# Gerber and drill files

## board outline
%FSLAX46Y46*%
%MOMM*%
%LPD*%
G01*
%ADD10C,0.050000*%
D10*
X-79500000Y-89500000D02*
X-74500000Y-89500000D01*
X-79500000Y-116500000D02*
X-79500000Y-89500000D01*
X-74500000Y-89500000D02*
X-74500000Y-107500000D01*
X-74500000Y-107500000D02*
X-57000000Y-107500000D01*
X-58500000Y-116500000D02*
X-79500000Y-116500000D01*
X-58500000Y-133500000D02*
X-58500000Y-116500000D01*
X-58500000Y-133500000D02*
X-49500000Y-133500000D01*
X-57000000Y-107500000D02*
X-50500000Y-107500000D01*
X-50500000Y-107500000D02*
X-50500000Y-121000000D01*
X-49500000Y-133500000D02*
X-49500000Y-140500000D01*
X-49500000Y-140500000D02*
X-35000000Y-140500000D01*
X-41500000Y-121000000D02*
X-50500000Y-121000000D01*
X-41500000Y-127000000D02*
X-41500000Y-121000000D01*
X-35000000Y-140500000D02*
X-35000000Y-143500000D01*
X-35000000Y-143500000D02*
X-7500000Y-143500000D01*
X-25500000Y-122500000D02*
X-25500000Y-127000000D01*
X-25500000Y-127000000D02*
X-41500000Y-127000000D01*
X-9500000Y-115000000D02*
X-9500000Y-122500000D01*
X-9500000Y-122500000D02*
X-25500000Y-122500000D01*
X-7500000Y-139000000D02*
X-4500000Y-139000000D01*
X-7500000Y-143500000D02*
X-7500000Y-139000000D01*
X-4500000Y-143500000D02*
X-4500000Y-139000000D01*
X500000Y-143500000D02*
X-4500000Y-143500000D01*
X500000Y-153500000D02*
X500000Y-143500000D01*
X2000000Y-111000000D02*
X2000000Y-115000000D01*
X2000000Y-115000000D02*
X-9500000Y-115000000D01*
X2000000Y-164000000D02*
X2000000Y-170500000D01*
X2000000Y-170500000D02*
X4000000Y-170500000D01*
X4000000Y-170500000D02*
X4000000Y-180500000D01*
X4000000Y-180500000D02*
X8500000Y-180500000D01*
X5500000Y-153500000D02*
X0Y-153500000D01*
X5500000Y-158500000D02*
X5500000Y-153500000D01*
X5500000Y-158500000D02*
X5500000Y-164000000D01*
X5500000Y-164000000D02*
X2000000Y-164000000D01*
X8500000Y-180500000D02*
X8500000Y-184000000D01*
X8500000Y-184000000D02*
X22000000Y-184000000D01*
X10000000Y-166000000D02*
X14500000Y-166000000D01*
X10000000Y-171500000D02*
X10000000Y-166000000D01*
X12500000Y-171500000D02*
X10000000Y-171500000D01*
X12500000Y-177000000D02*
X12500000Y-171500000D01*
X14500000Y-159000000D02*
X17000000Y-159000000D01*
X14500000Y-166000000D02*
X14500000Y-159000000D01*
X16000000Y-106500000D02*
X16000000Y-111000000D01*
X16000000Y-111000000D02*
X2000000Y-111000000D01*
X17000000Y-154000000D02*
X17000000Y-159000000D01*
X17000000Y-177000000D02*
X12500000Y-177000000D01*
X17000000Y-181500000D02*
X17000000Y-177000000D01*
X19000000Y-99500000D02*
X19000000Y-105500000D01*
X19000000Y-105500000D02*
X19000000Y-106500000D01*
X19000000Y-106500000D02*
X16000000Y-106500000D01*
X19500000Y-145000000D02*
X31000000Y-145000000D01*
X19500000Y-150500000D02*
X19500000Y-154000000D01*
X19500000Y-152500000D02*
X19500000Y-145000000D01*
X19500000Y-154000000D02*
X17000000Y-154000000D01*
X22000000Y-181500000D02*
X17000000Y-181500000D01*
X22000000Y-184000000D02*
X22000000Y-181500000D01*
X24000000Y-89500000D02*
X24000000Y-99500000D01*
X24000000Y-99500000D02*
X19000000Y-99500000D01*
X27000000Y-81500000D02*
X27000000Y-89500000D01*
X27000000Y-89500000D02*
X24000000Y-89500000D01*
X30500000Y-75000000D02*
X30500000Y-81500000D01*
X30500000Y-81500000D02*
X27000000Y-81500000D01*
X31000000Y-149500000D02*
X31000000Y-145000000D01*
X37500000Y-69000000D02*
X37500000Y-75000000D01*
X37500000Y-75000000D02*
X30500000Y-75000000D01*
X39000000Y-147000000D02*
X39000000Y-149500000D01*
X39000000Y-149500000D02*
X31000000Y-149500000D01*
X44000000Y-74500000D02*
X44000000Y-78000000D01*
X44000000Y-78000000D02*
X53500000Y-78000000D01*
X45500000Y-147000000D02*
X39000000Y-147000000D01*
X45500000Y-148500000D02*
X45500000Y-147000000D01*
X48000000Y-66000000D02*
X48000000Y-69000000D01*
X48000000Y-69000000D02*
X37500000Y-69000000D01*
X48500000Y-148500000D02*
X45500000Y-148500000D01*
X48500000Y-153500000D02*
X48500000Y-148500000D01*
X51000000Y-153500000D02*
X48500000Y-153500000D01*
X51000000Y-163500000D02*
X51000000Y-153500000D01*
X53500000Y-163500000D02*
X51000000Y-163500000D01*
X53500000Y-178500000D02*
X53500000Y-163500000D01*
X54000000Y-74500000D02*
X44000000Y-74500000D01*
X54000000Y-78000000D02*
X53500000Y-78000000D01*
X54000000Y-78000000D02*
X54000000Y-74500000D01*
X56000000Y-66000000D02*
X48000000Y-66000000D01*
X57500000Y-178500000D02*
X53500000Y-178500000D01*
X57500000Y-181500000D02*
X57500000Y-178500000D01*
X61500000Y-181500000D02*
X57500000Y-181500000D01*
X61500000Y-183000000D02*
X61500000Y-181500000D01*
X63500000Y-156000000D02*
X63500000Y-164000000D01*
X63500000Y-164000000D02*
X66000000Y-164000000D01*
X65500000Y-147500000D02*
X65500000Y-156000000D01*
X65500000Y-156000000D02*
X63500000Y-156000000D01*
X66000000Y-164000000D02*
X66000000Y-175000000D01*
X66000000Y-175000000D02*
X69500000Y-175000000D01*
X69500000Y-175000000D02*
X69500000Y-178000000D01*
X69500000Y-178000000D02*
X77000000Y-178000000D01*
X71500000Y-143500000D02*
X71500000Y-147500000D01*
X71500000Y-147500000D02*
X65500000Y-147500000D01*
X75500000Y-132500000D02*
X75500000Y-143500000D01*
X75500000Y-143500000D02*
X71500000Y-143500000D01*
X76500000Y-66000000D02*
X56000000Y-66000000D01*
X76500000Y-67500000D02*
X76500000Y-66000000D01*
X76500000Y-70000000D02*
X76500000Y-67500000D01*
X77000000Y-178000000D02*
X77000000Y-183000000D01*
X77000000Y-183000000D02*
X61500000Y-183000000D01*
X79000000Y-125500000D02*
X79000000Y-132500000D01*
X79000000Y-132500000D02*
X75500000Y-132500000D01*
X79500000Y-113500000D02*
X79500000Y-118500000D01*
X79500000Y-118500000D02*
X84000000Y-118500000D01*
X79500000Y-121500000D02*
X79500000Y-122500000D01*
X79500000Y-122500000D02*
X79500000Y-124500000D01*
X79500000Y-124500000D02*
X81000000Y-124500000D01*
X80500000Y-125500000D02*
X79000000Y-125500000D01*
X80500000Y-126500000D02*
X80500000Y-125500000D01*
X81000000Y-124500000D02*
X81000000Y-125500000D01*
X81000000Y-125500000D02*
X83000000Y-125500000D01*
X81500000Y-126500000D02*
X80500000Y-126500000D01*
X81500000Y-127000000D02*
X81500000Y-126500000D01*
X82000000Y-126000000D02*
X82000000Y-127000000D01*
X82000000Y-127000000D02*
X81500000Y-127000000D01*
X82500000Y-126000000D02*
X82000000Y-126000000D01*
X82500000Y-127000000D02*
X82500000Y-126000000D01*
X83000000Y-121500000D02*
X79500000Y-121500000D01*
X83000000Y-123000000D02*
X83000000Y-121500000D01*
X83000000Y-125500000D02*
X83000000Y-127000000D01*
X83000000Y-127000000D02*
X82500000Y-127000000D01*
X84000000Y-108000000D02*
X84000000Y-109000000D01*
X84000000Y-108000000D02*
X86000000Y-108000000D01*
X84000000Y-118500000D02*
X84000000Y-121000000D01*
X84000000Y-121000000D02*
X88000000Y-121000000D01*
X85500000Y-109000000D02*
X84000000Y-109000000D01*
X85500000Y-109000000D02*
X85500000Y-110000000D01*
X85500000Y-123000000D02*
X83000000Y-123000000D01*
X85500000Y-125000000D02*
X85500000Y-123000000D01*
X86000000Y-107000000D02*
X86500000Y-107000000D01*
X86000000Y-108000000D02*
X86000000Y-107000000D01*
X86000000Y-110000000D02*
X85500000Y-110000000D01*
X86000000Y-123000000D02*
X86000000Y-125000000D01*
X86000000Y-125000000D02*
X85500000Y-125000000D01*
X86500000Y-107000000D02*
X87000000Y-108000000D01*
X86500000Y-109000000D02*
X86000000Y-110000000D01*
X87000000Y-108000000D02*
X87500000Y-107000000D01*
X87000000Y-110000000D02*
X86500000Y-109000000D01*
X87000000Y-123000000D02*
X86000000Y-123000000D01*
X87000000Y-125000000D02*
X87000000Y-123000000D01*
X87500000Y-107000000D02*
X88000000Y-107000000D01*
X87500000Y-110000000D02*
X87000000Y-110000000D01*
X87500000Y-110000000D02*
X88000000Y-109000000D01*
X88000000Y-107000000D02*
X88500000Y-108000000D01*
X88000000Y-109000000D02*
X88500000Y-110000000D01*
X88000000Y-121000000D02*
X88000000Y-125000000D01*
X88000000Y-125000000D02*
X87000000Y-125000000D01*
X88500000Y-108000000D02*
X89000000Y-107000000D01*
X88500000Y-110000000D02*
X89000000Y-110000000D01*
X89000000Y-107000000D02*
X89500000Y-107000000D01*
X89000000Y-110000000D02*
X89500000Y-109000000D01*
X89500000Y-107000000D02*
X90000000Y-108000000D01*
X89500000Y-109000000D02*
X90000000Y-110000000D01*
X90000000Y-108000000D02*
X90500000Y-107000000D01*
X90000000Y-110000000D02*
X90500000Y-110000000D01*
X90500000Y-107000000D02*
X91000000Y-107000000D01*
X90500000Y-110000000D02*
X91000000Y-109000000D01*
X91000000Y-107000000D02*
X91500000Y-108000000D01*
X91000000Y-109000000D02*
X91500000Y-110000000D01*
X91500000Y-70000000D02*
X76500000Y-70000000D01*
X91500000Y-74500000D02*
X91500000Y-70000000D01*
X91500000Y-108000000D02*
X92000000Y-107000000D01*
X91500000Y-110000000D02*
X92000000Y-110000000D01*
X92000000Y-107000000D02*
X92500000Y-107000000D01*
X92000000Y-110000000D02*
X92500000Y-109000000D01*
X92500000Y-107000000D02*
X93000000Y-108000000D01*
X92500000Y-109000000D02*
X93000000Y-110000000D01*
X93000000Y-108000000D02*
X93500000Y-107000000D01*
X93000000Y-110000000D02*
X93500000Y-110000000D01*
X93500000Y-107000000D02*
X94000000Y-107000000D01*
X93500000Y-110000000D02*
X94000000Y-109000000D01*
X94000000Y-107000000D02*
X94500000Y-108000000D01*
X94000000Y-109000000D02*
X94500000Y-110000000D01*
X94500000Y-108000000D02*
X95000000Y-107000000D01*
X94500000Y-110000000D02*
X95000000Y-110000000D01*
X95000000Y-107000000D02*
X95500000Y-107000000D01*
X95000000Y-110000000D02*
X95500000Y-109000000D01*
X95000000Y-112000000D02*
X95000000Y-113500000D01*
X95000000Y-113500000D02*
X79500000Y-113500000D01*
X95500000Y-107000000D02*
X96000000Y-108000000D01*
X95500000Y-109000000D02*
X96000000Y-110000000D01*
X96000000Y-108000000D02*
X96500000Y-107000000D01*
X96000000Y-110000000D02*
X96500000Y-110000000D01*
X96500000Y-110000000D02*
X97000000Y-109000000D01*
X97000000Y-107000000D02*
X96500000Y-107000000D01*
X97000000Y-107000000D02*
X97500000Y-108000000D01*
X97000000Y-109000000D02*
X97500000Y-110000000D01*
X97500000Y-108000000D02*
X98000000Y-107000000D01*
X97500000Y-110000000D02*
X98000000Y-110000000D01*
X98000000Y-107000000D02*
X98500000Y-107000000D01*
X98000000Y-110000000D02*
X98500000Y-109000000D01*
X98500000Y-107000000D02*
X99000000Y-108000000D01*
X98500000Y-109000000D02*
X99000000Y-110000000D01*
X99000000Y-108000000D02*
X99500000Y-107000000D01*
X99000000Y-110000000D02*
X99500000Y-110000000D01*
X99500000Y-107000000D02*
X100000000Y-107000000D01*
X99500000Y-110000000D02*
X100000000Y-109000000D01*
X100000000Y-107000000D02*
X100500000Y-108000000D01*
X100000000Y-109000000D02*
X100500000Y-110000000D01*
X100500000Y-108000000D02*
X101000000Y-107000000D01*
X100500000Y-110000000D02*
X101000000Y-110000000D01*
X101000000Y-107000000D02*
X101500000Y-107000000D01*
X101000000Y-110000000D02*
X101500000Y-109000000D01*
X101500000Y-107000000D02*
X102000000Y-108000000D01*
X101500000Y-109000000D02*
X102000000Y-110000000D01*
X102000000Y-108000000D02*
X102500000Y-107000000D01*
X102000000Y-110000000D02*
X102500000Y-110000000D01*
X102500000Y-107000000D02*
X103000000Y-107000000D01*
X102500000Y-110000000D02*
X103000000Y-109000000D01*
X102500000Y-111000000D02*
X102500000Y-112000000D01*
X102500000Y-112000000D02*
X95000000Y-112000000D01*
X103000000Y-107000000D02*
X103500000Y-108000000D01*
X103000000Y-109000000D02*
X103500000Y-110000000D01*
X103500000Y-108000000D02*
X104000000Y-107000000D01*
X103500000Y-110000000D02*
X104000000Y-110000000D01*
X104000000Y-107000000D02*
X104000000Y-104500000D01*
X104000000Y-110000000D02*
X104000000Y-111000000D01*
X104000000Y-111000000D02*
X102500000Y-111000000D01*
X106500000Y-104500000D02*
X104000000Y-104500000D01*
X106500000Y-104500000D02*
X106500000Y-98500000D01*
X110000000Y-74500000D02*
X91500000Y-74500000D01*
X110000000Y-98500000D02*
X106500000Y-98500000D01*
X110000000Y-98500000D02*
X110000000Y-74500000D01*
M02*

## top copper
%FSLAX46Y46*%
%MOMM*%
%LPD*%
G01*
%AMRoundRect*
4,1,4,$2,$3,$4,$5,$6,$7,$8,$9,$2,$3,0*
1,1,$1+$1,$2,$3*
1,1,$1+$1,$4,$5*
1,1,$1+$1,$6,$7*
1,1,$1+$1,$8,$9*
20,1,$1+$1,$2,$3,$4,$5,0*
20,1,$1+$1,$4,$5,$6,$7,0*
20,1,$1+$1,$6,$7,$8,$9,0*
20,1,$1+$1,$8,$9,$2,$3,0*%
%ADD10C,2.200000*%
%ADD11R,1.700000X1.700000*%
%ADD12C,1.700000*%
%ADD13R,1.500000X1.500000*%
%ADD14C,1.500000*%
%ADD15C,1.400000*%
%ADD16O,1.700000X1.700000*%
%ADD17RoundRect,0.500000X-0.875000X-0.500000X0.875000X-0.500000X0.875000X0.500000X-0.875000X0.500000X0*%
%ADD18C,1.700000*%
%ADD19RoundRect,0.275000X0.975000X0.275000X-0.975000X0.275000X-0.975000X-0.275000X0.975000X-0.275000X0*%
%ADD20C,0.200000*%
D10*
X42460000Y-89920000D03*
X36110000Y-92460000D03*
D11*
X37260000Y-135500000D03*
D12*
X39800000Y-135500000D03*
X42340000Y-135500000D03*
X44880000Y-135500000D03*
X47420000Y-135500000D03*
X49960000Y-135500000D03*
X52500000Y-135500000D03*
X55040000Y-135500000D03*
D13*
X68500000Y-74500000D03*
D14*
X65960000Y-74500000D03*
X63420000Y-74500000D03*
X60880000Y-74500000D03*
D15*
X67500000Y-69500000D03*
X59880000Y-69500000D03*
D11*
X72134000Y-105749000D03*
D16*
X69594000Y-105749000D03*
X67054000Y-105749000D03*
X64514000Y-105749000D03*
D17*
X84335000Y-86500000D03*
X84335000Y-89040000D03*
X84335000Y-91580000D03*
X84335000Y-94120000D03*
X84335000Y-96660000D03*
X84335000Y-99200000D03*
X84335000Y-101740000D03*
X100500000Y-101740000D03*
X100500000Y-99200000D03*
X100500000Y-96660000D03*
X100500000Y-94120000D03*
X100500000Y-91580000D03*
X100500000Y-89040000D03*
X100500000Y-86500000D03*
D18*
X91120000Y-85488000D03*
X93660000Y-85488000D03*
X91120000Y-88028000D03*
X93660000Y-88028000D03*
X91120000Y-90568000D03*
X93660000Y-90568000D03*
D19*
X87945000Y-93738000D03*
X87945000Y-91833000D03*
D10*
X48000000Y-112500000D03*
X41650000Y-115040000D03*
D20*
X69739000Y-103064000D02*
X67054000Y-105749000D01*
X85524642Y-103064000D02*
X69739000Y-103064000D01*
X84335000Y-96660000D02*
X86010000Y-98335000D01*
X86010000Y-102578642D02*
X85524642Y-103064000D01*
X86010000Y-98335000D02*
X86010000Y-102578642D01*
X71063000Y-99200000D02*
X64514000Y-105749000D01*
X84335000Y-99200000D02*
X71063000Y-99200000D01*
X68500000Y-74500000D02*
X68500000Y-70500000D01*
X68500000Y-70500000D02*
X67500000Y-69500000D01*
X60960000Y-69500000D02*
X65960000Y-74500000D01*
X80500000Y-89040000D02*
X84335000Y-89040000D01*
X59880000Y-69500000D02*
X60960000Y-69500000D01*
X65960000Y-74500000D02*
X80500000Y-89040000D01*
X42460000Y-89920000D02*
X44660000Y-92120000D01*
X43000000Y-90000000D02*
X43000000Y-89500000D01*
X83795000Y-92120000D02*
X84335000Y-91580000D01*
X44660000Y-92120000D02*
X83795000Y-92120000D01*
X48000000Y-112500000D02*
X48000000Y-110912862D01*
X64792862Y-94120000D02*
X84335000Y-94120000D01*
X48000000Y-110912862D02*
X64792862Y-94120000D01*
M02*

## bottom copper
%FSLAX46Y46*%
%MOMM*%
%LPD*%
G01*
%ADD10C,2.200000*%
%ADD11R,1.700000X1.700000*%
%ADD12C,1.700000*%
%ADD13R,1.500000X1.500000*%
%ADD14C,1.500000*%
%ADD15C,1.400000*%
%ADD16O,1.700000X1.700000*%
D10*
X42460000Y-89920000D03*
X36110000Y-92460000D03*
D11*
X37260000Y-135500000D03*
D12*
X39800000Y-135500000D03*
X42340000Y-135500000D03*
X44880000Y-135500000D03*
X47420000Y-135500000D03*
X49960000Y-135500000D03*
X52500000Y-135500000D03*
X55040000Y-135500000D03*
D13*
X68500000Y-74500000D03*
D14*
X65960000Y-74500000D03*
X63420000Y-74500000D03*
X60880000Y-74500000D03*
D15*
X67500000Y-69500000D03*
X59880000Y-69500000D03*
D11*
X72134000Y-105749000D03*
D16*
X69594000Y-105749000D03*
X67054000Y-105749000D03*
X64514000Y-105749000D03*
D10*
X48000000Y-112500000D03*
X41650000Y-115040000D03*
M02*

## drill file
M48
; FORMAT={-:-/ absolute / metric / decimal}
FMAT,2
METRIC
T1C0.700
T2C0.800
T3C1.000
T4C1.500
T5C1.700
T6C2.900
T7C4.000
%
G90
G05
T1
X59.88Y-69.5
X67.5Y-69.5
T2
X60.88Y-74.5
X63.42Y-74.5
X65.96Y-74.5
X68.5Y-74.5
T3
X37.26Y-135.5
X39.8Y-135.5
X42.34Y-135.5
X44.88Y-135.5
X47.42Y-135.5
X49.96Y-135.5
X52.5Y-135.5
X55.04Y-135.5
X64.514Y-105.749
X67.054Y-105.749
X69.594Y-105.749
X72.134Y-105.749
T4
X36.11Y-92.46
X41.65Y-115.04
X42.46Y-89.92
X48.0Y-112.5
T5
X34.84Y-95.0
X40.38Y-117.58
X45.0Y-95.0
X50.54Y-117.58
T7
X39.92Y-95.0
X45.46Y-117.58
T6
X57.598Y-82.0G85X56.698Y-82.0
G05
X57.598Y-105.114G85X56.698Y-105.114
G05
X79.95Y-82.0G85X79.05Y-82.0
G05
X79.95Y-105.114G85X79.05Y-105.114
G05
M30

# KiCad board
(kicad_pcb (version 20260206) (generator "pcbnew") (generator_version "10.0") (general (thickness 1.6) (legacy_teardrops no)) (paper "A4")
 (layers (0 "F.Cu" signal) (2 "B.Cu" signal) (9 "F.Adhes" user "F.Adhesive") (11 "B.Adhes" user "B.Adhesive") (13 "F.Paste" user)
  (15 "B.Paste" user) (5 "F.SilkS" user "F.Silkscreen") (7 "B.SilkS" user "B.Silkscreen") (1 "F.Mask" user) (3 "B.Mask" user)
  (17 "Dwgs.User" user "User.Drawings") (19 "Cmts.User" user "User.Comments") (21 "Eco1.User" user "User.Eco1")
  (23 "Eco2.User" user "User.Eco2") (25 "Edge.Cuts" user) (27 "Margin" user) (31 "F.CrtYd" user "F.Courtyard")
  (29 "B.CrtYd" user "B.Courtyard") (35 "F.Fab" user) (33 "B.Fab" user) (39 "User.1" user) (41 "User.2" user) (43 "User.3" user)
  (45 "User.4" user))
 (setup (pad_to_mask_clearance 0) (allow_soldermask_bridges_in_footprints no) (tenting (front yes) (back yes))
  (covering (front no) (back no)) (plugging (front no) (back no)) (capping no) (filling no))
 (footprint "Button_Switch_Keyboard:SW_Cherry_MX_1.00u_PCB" (layer "F.Cu") (at 42.46 89.92)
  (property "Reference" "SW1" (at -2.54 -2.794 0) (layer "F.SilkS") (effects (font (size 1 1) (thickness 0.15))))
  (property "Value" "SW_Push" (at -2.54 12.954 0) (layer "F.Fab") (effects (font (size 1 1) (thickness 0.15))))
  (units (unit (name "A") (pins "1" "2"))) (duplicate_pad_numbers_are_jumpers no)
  (pad "" np_thru_hole circle (at -7.62 5.08) (size 1.7 1.7) (drill 1.7) (layers "*.Cu" "*.Mask"))
  (pad "" np_thru_hole circle (at -2.54 5.08) (size 4 4) (drill 4) (layers "*.Cu" "*.Mask"))
  (pad "" np_thru_hole circle (at 2.54 5.08) (size 1.7 1.7) (drill 1.7) (layers "*.Cu" "*.Mask"))
  (pad "1" thru_hole circle (at 0 0) (size 2.2 2.2) (drill 1.5) (layers "*.Cu" "*.Mask") (remove_unused_layers no) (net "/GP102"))
  (pad "2" thru_hole circle (at -6.35 2.54) (size 2.2 2.2) (drill 1.5) (layers "*.Cu" "*.Mask") (remove_unused_layers no) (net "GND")))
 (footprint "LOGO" (layer "F.Cu") (at 22 131)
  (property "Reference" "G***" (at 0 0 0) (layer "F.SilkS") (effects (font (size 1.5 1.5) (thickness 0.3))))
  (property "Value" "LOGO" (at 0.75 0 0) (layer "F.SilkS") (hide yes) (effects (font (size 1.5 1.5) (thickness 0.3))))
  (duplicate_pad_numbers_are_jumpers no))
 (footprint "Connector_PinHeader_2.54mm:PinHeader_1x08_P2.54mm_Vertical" (layer "F.Cu") (at 37.26 135.5 90)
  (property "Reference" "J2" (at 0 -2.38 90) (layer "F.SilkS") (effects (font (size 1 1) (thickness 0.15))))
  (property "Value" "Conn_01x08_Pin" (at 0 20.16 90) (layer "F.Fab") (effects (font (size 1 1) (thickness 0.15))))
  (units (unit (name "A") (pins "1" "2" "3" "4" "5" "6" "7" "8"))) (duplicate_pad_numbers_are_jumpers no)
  (pad "1" thru_hole rect (at 0 0 90) (size 1.7 1.7) (drill 1) (layers "*.Cu" "*.Mask") (remove_unused_layers no) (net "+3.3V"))
  (pad "2" thru_hole circle (at 0 2.54 90) (size 1.7 1.7) (drill 1) (layers "*.Cu" "*.Mask") (remove_unused_layers no) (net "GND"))
  (pad "3" thru_hole circle (at 0 5.08 90) (size 1.7 1.7) (drill 1) (layers "*.Cu" "*.Mask") (remove_unused_layers no) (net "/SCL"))
  (pad "4" thru_hole circle (at 0 7.62 90) (size 1.7 1.7) (drill 1) (layers "*.Cu" "*.Mask") (remove_unused_layers no) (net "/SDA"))
  (pad "5" thru_hole circle (at 0 10.16 90) (size 1.7 1.7) (drill 1) (layers "*.Cu" "*.Mask") (remove_unused_layers no)
   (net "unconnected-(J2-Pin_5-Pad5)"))
  (pad "6" thru_hole circle (at 0 12.7 90) (size 1.7 1.7) (drill 1) (layers "*.Cu" "*.Mask") (remove_unused_layers no)
   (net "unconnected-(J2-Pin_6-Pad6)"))
  (pad "7" thru_hole circle (at 0 15.24 90) (size 1.7 1.7) (drill 1) (layers "*.Cu" "*.Mask") (remove_unused_layers no)
   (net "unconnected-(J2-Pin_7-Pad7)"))
  (pad "8" thru_hole circle (at 0 17.78 90) (size 1.7 1.7) (drill 1) (layers "*.Cu" "*.Mask") (remove_unused_layers no)
   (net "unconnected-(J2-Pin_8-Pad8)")))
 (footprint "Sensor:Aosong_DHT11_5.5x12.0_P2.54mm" (layer "F.Cu") (at 68.5 74.5 -90)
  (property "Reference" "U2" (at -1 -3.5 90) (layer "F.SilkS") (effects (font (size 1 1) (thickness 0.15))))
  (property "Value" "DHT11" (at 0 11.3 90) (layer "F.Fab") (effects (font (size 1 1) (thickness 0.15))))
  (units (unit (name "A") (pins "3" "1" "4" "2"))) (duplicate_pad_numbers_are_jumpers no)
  (pad "1" thru_hole rect (at 0 0 270) (size 1.5 1.5) (drill 0.8) (layers "*.Cu" "*.Mask") (remove_unused_layers no) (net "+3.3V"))
  (pad "2" thru_hole circle (at 0 2.54 270) (size 1.5 1.5) (drill 0.8) (layers "*.Cu" "*.Mask") (remove_unused_layers no)
   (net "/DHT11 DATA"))
  (pad "3" thru_hole circle (at 0 5.08 270) (size 1.5 1.5) (drill 0.8) (layers "*.Cu" "*.Mask") (remove_unused_layers no)
   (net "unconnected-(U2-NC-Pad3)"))
  (pad "4" thru_hole circle (at 0 7.62 270) (size 1.5 1.5) (drill 0.8) (layers "*.Cu" "*.Mask") (remove_unused_layers no) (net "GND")))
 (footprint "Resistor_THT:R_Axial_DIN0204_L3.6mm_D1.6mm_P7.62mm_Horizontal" (layer "F.Cu") (at 67.5 69.5 180)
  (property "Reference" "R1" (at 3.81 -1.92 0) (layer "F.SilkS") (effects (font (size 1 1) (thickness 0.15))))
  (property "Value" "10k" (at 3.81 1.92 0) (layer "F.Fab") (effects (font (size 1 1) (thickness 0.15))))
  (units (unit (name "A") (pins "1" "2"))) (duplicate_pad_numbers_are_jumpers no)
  (pad "1" thru_hole circle (at 0 0 180) (size 1.4 1.4) (drill 0.7) (layers "*.Cu" "*.Mask") (remove_unused_layers no) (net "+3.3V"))
  (pad "2" thru_hole circle (at 7.62 0 180) (size 1.4 1.4) (drill 0.7) (layers "*.Cu" "*.Mask") (remove_unused_layers no)
   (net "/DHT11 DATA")))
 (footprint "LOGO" (layer "F.Cu") (at 68.5 121.5)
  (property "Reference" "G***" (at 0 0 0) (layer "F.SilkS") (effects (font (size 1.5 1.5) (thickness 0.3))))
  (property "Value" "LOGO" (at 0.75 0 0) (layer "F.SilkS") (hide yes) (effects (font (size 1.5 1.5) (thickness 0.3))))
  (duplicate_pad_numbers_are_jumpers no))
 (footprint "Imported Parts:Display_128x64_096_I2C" (layer "F.Cu") (at 68.324 105.749 180)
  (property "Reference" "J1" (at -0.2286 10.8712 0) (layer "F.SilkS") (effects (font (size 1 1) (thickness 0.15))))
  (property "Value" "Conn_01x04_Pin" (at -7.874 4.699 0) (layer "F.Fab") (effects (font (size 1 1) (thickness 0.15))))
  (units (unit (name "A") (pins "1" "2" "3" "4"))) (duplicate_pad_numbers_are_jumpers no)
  (pad "" np_thru_hole oval (at -11.176 0.635 180) (size 3.8 2.9) (drill oval 3.8 2.9) (layers "*.Cu" "*.Mask"))
  (pad "" np_thru_hole oval (at -11.176 23.749 180) (size 3.8 2.9) (drill oval 3.8 2.9) (layers "*.Cu" "*.Mask"))
  (pad "" np_thru_hole oval (at 11.176 0.635 180) (size 3.8 2.9) (drill oval 3.8 2.9) (layers "*.Cu" "*.Mask"))
  (pad "" np_thru_hole oval (at 11.176 23.749 180) (size 3.8 2.9) (drill oval 3.8 2.9) (layers "*.Cu" "*.Mask"))
  (pad "1" thru_hole rect (at -3.81 0 270) (size 1.7 1.7) (drill 1) (layers "*.Cu" "*.Mask") (remove_unused_layers no) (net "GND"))
  (pad "2" thru_hole oval (at -1.27 0 270) (size 1.7 1.7) (drill 1) (layers "*.Cu" "*.Mask") (remove_unused_layers no) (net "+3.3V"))
  (pad "3" thru_hole oval (at 1.27 0 270) (size 1.7 1.7) (drill 1) (layers "*.Cu" "*.Mask") (remove_unused_layers no) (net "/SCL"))
  (pad "4" thru_hole oval (at 3.81 0 270) (size 1.7 1.7) (drill 1) (layers "*.Cu" "*.Mask") (remove_unused_layers no) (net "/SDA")))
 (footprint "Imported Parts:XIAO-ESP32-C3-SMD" (layer "F.Cu") (at 83.5 104.62)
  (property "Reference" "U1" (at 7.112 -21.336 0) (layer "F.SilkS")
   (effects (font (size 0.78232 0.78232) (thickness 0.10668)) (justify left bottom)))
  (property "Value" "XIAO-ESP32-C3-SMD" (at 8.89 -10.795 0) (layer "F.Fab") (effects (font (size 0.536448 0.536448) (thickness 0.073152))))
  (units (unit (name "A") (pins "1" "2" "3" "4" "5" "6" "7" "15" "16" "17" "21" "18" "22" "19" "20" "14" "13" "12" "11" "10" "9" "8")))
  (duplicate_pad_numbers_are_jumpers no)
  (pad "1" smd roundrect (at 0.835 -18.12) (size 2.75 2) (layers "F.Cu" "F.Mask" "F.Paste") (roundrect_rratio 0.25)
   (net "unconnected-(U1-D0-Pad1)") (solder_mask_margin 0.0508) (thermal_bridge_angle 45))
  (pad "2" smd roundrect (at 0.835 -15.58) (size 2.75 2) (layers "F.Cu" "F.Mask" "F.Paste") (roundrect_rratio 0.25) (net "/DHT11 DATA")
   (solder_mask_margin 0.0508) (thermal_bridge_angle 45))
  (pad "3" smd roundrect (at 0.835 -13.04) (size 2.75 2) (layers "F.Cu" "F.Mask" "F.Paste") (roundrect_rratio 0.25) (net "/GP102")
   (solder_mask_margin 0.0508) (thermal_bridge_angle 45))
  (pad "4" smd roundrect (at 0.835 -10.5) (size 2.75 2) (layers "F.Cu" "F.Mask" "F.Paste") (roundrect_rratio 0.25) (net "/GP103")
   (solder_mask_margin 0.0508) (thermal_bridge_angle 45))
  (pad "5" smd roundrect (at 0.835 -7.96) (size 2.75 2) (layers "F.Cu" "F.Mask" "F.Paste") (roundrect_rratio 0.25) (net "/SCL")
   (solder_mask_margin 0.0508) (thermal_bridge_angle 45))
  (pad "6" smd roundrect (at 0.835 -5.42) (size 2.75 2) (layers "F.Cu" "F.Mask" "F.Paste") (roundrect_rratio 0.25) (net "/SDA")
   (solder_mask_margin 0.0508) (thermal_bridge_angle 45))
  (pad "7" smd roundrect (at 0.835 -2.88) (size 2.75 2) (layers "F.Cu" "F.Mask" "F.Paste") (roundrect_rratio 0.25)
   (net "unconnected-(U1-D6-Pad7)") (solder_mask_margin 0.0508) (thermal_bridge_angle 45))
  (pad "8" smd roundrect (at 17 -2.88) (size 2.75 2) (layers "F.Cu" "F.Mask" "F.Paste") (roundrect_rratio 0.25)
   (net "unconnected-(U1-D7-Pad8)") (solder_mask_margin 0.0508) (thermal_bridge_angle 45))
  (pad "9" smd roundrect (at 17 -5.42) (size 2.75 2) (layers "F.Cu" "F.Mask" "F.Paste") (roundrect_rratio 0.25)
   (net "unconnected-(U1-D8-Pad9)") (solder_mask_margin 0.0508) (thermal_bridge_angle 45))
  (pad "10" smd roundrect (at 17 -7.96) (size 2.75 2) (layers "F.Cu" "F.Mask" "F.Paste") (roundrect_rratio 0.25)
   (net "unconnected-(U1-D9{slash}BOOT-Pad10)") (solder_mask_margin 0.0508) (thermal_bridge_angle 45))
  (pad "11" smd roundrect (at 17 -10.5) (size 2.75 2) (layers "F.Cu" "F.Mask" "F.Paste") (roundrect_rratio 0.25)
   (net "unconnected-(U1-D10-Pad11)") (solder_mask_margin 0.0508) (thermal_bridge_angle 45))
  (pad "12" smd roundrect (at 17 -13.04) (size 2.75 2) (layers "F.Cu" "F.Mask" "F.Paste") (roundrect_rratio 0.25) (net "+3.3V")
   (solder_mask_margin 0.0508) (thermal_bridge_angle 45))
  (pad "13" smd roundrect (at 17 -15.58) (size 2.75 2) (layers "F.Cu" "F.Mask" "F.Paste") (roundrect_rratio 0.25) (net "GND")
   (solder_mask_margin 0.0508) (thermal_bridge_angle 45))
  (pad "14" smd roundrect (at 17 -18.12) (size 2.75 2) (layers "F.Cu" "F.Mask" "F.Paste") (roundrect_rratio 0.25) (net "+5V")
   (solder_mask_margin 0.0508) (thermal_bridge_angle 45))
  (pad "15" smd circle (at 7.62 -19.132) (size 1.7 1.7) (layers "F.Cu" "F.Mask" "F.Paste") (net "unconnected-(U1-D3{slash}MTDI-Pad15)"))
  (pad "16" smd circle (at 10.16 -19.132) (size 1.7 1.7) (layers "F.Cu" "F.Mask" "F.Paste") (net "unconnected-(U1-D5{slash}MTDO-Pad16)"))
  (pad "17" smd circle (at 7.62 -16.592) (size 1.7 1.7) (layers "F.Cu" "F.Mask" "F.Paste") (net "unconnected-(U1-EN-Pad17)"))
  (pad "18" smd circle (at 10.16 -16.592) (size 1.7 1.7) (layers "F.Cu" "F.Mask" "F.Paste") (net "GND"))
  (pad "19" smd circle (at 7.62 -14.052) (size 1.7 1.7) (layers "F.Cu" "F.Mask" "F.Paste") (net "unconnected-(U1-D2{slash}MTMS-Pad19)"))
  (pad "20" smd circle (at 10.16 -14.052) (size 1.7 1.7) (layers "F.Cu" "F.Mask" "F.Paste") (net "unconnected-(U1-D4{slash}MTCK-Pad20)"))
  (pad "21" smd roundrect (at 4.445 -10.882 180) (size 2.5 1.1) (layers "F.Cu" "F.Mask" "F.Paste") (roundrect_rratio 0.25)
   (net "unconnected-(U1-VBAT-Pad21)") (thermal_bridge_angle 45))
  (pad "22" smd roundrect (at 4.445 -12.787 180) (size 2.5 1.1) (layers "F.Cu" "F.Mask" "F.Paste") (roundrect_rratio 0.25)
   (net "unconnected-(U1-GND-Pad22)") (thermal_bridge_angle 45)))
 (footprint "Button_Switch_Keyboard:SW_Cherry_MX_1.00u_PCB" (layer "F.Cu") (at 48 112.5)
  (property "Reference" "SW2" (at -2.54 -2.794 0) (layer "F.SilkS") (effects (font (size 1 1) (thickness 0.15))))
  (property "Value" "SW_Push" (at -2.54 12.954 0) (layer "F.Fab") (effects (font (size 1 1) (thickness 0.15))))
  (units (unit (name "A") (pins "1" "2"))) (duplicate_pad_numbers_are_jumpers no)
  (pad "" np_thru_hole circle (at -7.62 5.08) (size 1.7 1.7) (drill 1.7) (layers "*.Cu" "*.Mask"))
  (pad "" np_thru_hole circle (at -2.54 5.08) (size 4 4) (drill 4) (layers "*.Cu" "*.Mask"))
  (pad "" np_thru_hole circle (at 2.54 5.08) (size 1.7 1.7) (drill 1.7) (layers "*.Cu" "*.Mask"))
  (pad "1" thru_hole circle (at 0 0) (size 2.2 2.2) (drill 1.5) (layers "*.Cu" "*.Mask") (remove_unused_layers no) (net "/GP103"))
  (pad "2" thru_hole circle (at -6.35 2.54) (size 2.2 2.2) (drill 1.5) (layers "*.Cu" "*.Mask") (remove_unused_layers no) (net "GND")))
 (gr_line (start -79.5 89.5) (end -74.5 89.5) (stroke (width 0.05) (type default)) (layer "Edge.Cuts"))
 (gr_line (start -79.5 116.5) (end -79.5 89.5) (stroke (width 0.05) (type default)) (layer "Edge.Cuts"))
 (gr_line (start -74.5 89.5) (end -74.5 107.5) (stroke (width 0.05) (type default)) (layer "Edge.Cuts"))
 (gr_line (start -74.5 107.5) (end -57 107.5) (stroke (width 0.05) (type default)) (layer "Edge.Cuts"))
 (gr_line (start -58.5 116.5) (end -79.5 116.5) (stroke (width 0.05) (type default)) (layer "Edge.Cuts"))
 (gr_line (start -58.5 133.5) (end -58.5 116.5) (stroke (width 0.05) (type default)) (layer "Edge.Cuts"))
 (gr_line (start -58.5 133.5) (end -49.5 133.5) (stroke (width 0.05) (type default)) (layer "Edge.Cuts"))
 (gr_line (start -57 107.5) (end -50.5 107.5) (stroke (width 0.05) (type default)) (layer "Edge.Cuts"))
 (gr_line (start -50.5 107.5) (end -50.5 121) (stroke (width 0.05) (type default)) (layer "Edge.Cuts"))
 (gr_line (start -49.5 133.5) (end -49.5 140.5) (stroke (width 0.05) (type default)) (layer "Edge.Cuts"))
 (gr_line (start -49.5 140.5) (end -35 140.5) (stroke (width 0.05) (type default)) (layer "Edge.Cuts"))
 (gr_line (start -41.5 121) (end -50.5 121) (stroke (width 0.05) (type default)) (layer "Edge.Cuts"))
 (gr_line (start -41.5 127) (end -41.5 121) (stroke (width 0.05) (type default)) (layer "Edge.Cuts"))
 (gr_line (start -35 140.5) (end -35 143.5) (stroke (width 0.05) (type default)) (layer "Edge.Cuts"))
 (gr_line (start -35 143.5) (end -7.5 143.5) (stroke (width 0.05) (type default)) (layer "Edge.Cuts"))
 (gr_line (start -25.5 122.5) (end -25.5 127) (stroke (width 0.05) (type default)) (layer "Edge.Cuts"))
 (gr_line (start -25.5 127) (end -41.5 127) (stroke (width 0.05) (type default)) (layer "Edge.Cuts"))
 (gr_line (start -9.5 115) (end -9.5 122.5) (stroke (width 0.05) (type default)) (layer "Edge.Cuts"))
 (gr_line (start -9.5 122.5) (end -25.5 122.5) (stroke (width 0.05) (type default)) (layer "Edge.Cuts"))
 (gr_line (start -7.5 139) (end -4.5 139) (stroke (width 0.05) (type default)) (layer "Edge.Cuts"))
 (gr_line (start -7.5 143.5) (end -7.5 139) (stroke (width 0.05) (type default)) (layer "Edge.Cuts"))
 (gr_line (start -4.5 143.5) (end -4.5 139) (stroke (width 0.05) (type default)) (layer "Edge.Cuts"))
 (gr_line (start 0.5 143.5) (end -4.5 143.5) (stroke (width 0.05) (type default)) (layer "Edge.Cuts"))
 (gr_line (start 0.5 153.5) (end 0.5 143.5) (stroke (width 0.05) (type default)) (layer "Edge.Cuts"))
 (gr_line (start 2 111) (end 2 115) (stroke (width 0.05) (type default)) (layer "Edge.Cuts"))
 (gr_line (start 2 115) (end -9.5 115) (stroke (width 0.05) (type default)) (layer "Edge.Cuts"))
 (gr_line (start 2 164) (end 2 170.5) (stroke (width 0.05) (type default)) (layer "Edge.Cuts"))
 (gr_line (start 2 170.5) (end 4 170.5) (stroke (width 0.05) (type default)) (layer "Edge.Cuts"))
 (gr_line (start 4 170.5) (end 4 180.5) (stroke (width 0.05) (type default)) (layer "Edge.Cuts"))
 (gr_line (start 4 180.5) (end 8.5 180.5) (stroke (width 0.05) (type default)) (layer "Edge.Cuts"))
 (gr_line (start 5.5 153.5) (end 0 153.5) (stroke (width 0.05) (type default)) (layer "Edge.Cuts"))
 (gr_line (start 5.5 158.5) (end 5.5 153.5) (stroke (width 0.05) (type default)) (layer "Edge.Cuts"))
 (gr_line (start 5.5 158.5) (end 5.5 164) (stroke (width 0.05) (type default)) (layer "Edge.Cuts"))
 (gr_line (start 5.5 164) (end 2 164) (stroke (width 0.05) (type default)) (layer "Edge.Cuts"))
 (gr_line (start 8.5 180.5) (end 8.5 184) (stroke (width 0.05) (type default)) (layer "Edge.Cuts"))
 (gr_line (start 8.5 184) (end 22 184) (stroke (width 0.05) (type default)) (layer "Edge.Cuts"))
 (gr_line (start 10 166) (end 14.5 166) (stroke (width 0.05) (type default)) (layer "Edge.Cuts"))
 (gr_line (start 10 171.5) (end 10 166) (stroke (width 0.05) (type default)) (layer "Edge.Cuts"))
 (gr_line (start 12.5 171.5) (end 10 171.5) (stroke (width 0.05) (type default)) (layer "Edge.Cuts"))
 (gr_line (start 12.5 177) (end 12.5 171.5) (stroke (width 0.05) (type default)) (layer "Edge.Cuts"))
 (gr_line (start 14.5 159) (end 17 159) (stroke (width 0.05) (type default)) (layer "Edge.Cuts"))
 (gr_line (start 14.5 166) (end 14.5 159) (stroke (width 0.05) (type default)) (layer "Edge.Cuts"))
 (gr_line (start 16 106.5) (end 16 111) (stroke (width 0.05) (type default)) (layer "Edge.Cuts"))
 (gr_line (start 16 111) (end 2 111) (stroke (width 0.05) (type default)) (layer "Edge.Cuts"))
 (gr_line (start 17 154) (end 17 159) (stroke (width 0.05) (type default)) (layer "Edge.Cuts"))
 (gr_line (start 17 177) (end 12.5 177) (stroke (width 0.05) (type default)) (layer "Edge.Cuts"))
 (gr_line (start 17 181.5) (end 17 177) (stroke (width 0.05) (type default)) (layer "Edge.Cuts"))
 (gr_line (start 19 99.5) (end 19 105.5) (stroke (width 0.05) (type default)) (layer "Edge.Cuts"))
 (gr_line (start 19 105.5) (end 19 106.5) (stroke (width 0.05) (type default)) (layer "Edge.Cuts"))
 (gr_line (start 19 106.5) (end 16 106.5) (stroke (width 0.05) (type default)) (layer "Edge.Cuts"))
 (gr_line (start 19.5 145) (end 31 145) (stroke (width 0.05) (type default)) (layer "Edge.Cuts"))
 (gr_line (start 19.5 150.5) (end 19.5 154) (stroke (width 0.05) (type default)) (layer "Edge.Cuts"))
 (gr_line (start 19.5 152.5) (end 19.5 145) (stroke (width 0.05) (type default)) (layer "Edge.Cuts"))
 (gr_line (start 19.5 154) (end 17 154) (stroke (width 0.05) (type default)) (layer "Edge.Cuts"))
 (gr_line (start 22 181.5) (end 17 181.5) (stroke (width 0.05) (type default)) (layer "Edge.Cuts"))
 (gr_line (start 22 184) (end 22 181.5) (stroke (width 0.05) (type default)) (layer "Edge.Cuts"))
 (gr_line (start 24 89.5) (end 24 99.5) (stroke (width 0.05) (type default)) (layer "Edge.Cuts"))
 (gr_line (start 24 99.5) (end 19 99.5) (stroke (width 0.05) (type default)) (layer "Edge.Cuts"))
 (gr_line (start 27 81.5) (end 27 89.5) (stroke (width 0.05) (type default)) (layer "Edge.Cuts"))
 (gr_line (start 27 89.5) (end 24 89.5) (stroke (width 0.05) (type default)) (layer "Edge.Cuts"))
 (gr_line (start 30.5 75) (end 30.5 81.5) (stroke (width 0.05) (type default)) (layer "Edge.Cuts"))
 (gr_line (start 30.5 81.5) (end 27 81.5) (stroke (width 0.05) (type default)) (layer "Edge.Cuts"))
 (gr_line (start 31 149.5) (end 31 145) (stroke (width 0.05) (type default)) (layer "Edge.Cuts"))
 (gr_line (start 37.5 69) (end 37.5 75) (stroke (width 0.05) (type default)) (layer "Edge.Cuts"))
 (gr_line (start 37.5 75) (end 30.5 75) (stroke (width 0.05) (type default)) (layer "Edge.Cuts"))
 (gr_line (start 39 147) (end 39 149.5) (stroke (width 0.05) (type default)) (layer "Edge.Cuts"))
 (gr_line (start 39 149.5) (end 31 149.5) (stroke (width 0.05) (type default)) (layer "Edge.Cuts"))
 (gr_line (start 44 74.5) (end 44 78) (stroke (width 0.05) (type default)) (layer "Edge.Cuts"))
 (gr_line (start 44 78) (end 53.5 78) (stroke (width 0.05) (type default)) (layer "Edge.Cuts"))
 (gr_line (start 45.5 147) (end 39 147) (stroke (width 0.05) (type default)) (layer "Edge.Cuts"))
 (gr_line (start 45.5 148.5) (end 45.5 147) (stroke (width 0.05) (type default)) (layer "Edge.Cuts"))
 (gr_line (start 48 66) (end 48 69) (stroke (width 0.05) (type default)) (layer "Edge.Cuts"))
 (gr_line (start 48 69) (end 37.5 69) (stroke (width 0.05) (type default)) (layer "Edge.Cuts"))
 (gr_line (start 48.5 148.5) (end 45.5 148.5) (stroke (width 0.05) (type default)) (layer "Edge.Cuts"))
 (gr_line (start 48.5 153.5) (end 48.5 148.5) (stroke (width 0.05) (type default)) (layer "Edge.Cuts"))
 (gr_line (start 51 153.5) (end 48.5 153.5) (stroke (width 0.05) (type default)) (layer "Edge.Cuts"))
 (gr_line (start 51 163.5) (end 51 153.5) (stroke (width 0.05) (type default)) (layer "Edge.Cuts"))
 (gr_line (start 53.5 163.5) (end 51 163.5) (stroke (width 0.05) (type default)) (layer "Edge.Cuts"))
 (gr_line (start 53.5 178.5) (end 53.5 163.5) (stroke (width 0.05) (type default)) (layer "Edge.Cuts"))
 (gr_line (start 54 74.5) (end 44 74.5) (stroke (width 0.05) (type default)) (layer "Edge.Cuts"))
 (gr_line (start 54 78) (end 53.5 78) (stroke (width 0.05) (type default)) (layer "Edge.Cuts"))
 (gr_line (start 54 78) (end 54 74.5) (stroke (width 0.05) (type default)) (layer "Edge.Cuts"))
 (gr_line (start 56 66) (end 48 66) (stroke (width 0.05) (type default)) (layer "Edge.Cuts"))
 (gr_line (start 57.5 178.5) (end 53.5 178.5) (stroke (width 0.05) (type default)) (layer "Edge.Cuts"))
 (gr_line (start 57.5 181.5) (end 57.5 178.5) (stroke (width 0.05) (type default)) (layer "Edge.Cuts"))
 (gr_line (start 61.5 181.5) (end 57.5 181.5) (stroke (width 0.05) (type default)) (layer "Edge.Cuts"))
 (gr_line (start 61.5 183) (end 61.5 181.5) (stroke (width 0.05) (type default)) (layer "Edge.Cuts"))
 (gr_line (start 63.5 156) (end 63.5 164) (stroke (width 0.05) (type default)) (layer "Edge.Cuts"))
 (gr_line (start 63.5 164) (end 66 164) (stroke (width 0.05) (type default)) (layer "Edge.Cuts"))
 (gr_line (start 65.5 147.5) (end 65.5 156) (stroke (width 0.05) (type default)) (layer "Edge.Cuts"))
 (gr_line (start 65.5 156) (end 63.5 156) (stroke (width 0.05) (type default)) (layer "Edge.Cuts"))
 (gr_line (start 66 164) (end 66 175) (stroke (width 0.05) (type default)) (layer "Edge.Cuts"))
 (gr_line (start 66 175) (end 69.5 175) (stroke (width 0.05) (type default)) (layer "Edge.Cuts"))
 (gr_line (start 69.5 175) (end 69.5 178) (stroke (width 0.05) (type default)) (layer "Edge.Cuts"))
 (gr_line (start 69.5 178) (end 77 178) (stroke (width 0.05) (type default)) (layer "Edge.Cuts"))
 (gr_line (start 71.5 143.5) (end 71.5 147.5) (stroke (width 0.05) (type default)) (layer "Edge.Cuts"))
 (gr_line (start 71.5 147.5) (end 65.5 147.5) (stroke (width 0.05) (type default)) (layer "Edge.Cuts"))
 (gr_line (start 75.5 132.5) (end 75.5 143.5) (stroke (width 0.05) (type default)) (layer "Edge.Cuts"))
 (gr_line (start 75.5 143.5) (end 71.5 143.5) (stroke (width 0.05) (type default)) (layer "Edge.Cuts"))
 (gr_line (start 76.5 66) (end 56 66) (stroke (width 0.05) (type default)) (layer "Edge.Cuts"))
 (gr_line (start 76.5 67.5) (end 76.5 66) (stroke (width 0.05) (type default)) (layer "Edge.Cuts"))
 (gr_line (start 76.5 70) (end 76.5 67.5) (stroke (width 0.05) (type default)) (layer "Edge.Cuts"))
 (gr_line (start 77 178) (end 77 183) (stroke (width 0.05) (type default)) (layer "Edge.Cuts"))
 (gr_line (start 77 183) (end 61.5 183) (stroke (width 0.05) (type default)) (layer "Edge.Cuts"))
 (gr_line (start 79 125.5) (end 79 132.5) (stroke (width 0.05) (type default)) (layer "Edge.Cuts"))
 (gr_line (start 79 132.5) (end 75.5 132.5) (stroke (width 0.05) (type default)) (layer "Edge.Cuts"))
 (gr_line (start 79.5 113.5) (end 79.5 118.5) (stroke (width 0.05) (type default)) (layer "Edge.Cuts"))
 (gr_line (start 79.5 118.5) (end 84 118.5) (stroke (width 0.05) (type default)) (layer "Edge.Cuts"))
 (gr_line (start 79.5 121.5) (end 79.5 122.5) (stroke (width 0.05) (type default)) (layer "Edge.Cuts"))
 (gr_line (start 79.5 122.5) (end 79.5 124.5) (stroke (width 0.05) (type default)) (layer "Edge.Cuts"))
 (gr_line (start 79.5 124.5) (end 81 124.5) (stroke (width 0.05) (type default)) (layer "Edge.Cuts"))
 (gr_line (start 80.5 125.5) (end 79 125.5) (stroke (width 0.05) (type default)) (layer "Edge.Cuts"))
 (gr_line (start 80.5 126.5) (end 80.5 125.5) (stroke (width 0.05) (type default)) (layer "Edge.Cuts"))
 (gr_line (start 81 124.5) (end 81 125.5) (stroke (width 0.05) (type default)) (layer "Edge.Cuts"))
 (gr_line (start 81 125.5) (end 83 125.5) (stroke (width 0.05) (type default)) (layer "Edge.Cuts"))
 (gr_line (start 81.5 126.5) (end 80.5 126.5) (stroke (width 0.05) (type default)) (layer "Edge.Cuts"))
 (gr_line (start 81.5 127) (end 81.5 126.5) (stroke (width 0.05) (type default)) (layer "Edge.Cuts"))
 (gr_line (start 82 126) (end 82 127) (stroke (width 0.05) (type default)) (layer "Edge.Cuts"))
 (gr_line (start 82 127) (end 81.5 127) (stroke (width 0.05) (type default)) (layer "Edge.Cuts"))
 (gr_line (start 82.5 126) (end 82 126) (stroke (width 0.05) (type default)) (layer "Edge.Cuts"))
 (gr_line (start 82.5 127) (end 82.5 126) (stroke (width 0.05) (type default)) (layer "Edge.Cuts"))
 (gr_line (start 83 121.5) (end 79.5 121.5) (stroke (width 0.05) (type default)) (layer "Edge.Cuts"))
 (gr_line (start 83 123) (end 83 121.5) (stroke (width 0.05) (type default)) (layer "Edge.Cuts"))
 (gr_line (start 83 125.5) (end 83 127) (stroke (width 0.05) (type default)) (layer "Edge.Cuts"))
 (gr_line (start 83 127) (end 82.5 127) (stroke (width 0.05) (type default)) (layer "Edge.Cuts"))
 (gr_line (start 84 108) (end 84 109) (stroke (width 0.05) (type default)) (layer "Edge.Cuts"))
 (gr_line (start 84 108) (end 86 108) (stroke (width 0.05) (type default)) (layer "Edge.Cuts"))
 (gr_line (start 84 118.5) (end 84 121) (stroke (width 0.05) (type default)) (layer "Edge.Cuts"))
 (gr_line (start 84 121) (end 88 121) (stroke (width 0.05) (type default)) (layer "Edge.Cuts"))
 (gr_line (start 85.5 109) (end 84 109) (stroke (width 0.05) (type default)) (layer "Edge.Cuts"))
 (gr_line (start 85.5 109) (end 85.5 110) (stroke (width 0.05) (type default)) (layer "Edge.Cuts"))
 (gr_line (start 85.5 123) (end 83 123) (stroke (width 0.05) (type default)) (layer "Edge.Cuts"))
 (gr_line (start 85.5 125) (end 85.5 123) (stroke (width 0.05) (type default)) (layer "Edge.Cuts"))
 (gr_line (start 86 107) (end 86.5 107) (stroke (width 0.05) (type default)) (layer "Edge.Cuts"))
 (gr_line (start 86 108) (end 86 107) (stroke (width 0.05) (type default)) (layer "Edge.Cuts"))
 (gr_line (start 86 110) (end 85.5 110) (stroke (width 0.05) (type default)) (layer "Edge.Cuts"))
 (gr_line (start 86 123) (end 86 125) (stroke (width 0.05) (type default)) (layer "Edge.Cuts"))
 (gr_line (start 86 125) (end 85.5 125) (stroke (width 0.05) (type default)) (layer "Edge.Cuts"))
 (gr_line (start 86.5 107) (end 87 108) (stroke (width 0.05) (type default)) (layer "Edge.Cuts"))
 (gr_line (start 86.5 109) (end 86 110) (stroke (width 0.05) (type default)) (layer "Edge.Cuts"))
 (gr_line (start 87 108) (end 87.5 107) (stroke (width 0.05) (type default)) (layer "Edge.Cuts"))
 (gr_line (start 87 110) (end 86.5 109) (stroke (width 0.05) (type default)) (layer "Edge.Cuts"))
 (gr_line (start 87 123) (end 86 123) (stroke (width 0.05) (type default)) (layer "Edge.Cuts"))
 (gr_line (start 87 125) (end 87 123) (stroke (width 0.05) (type default)) (layer "Edge.Cuts"))
 (gr_line (start 87.5 107) (end 88 107) (stroke (width 0.05) (type default)) (layer "Edge.Cuts"))
 (gr_line (start 87.5 110) (end 87 110) (stroke (width 0.05) (type default)) (layer "Edge.Cuts"))
 (gr_line (start 87.5 110) (end 88 109) (stroke (width 0.05) (type default)) (layer "Edge.Cuts"))
 (gr_line (start 88 107) (end 88.5 108) (stroke (width 0.05) (type default)) (layer "Edge.Cuts"))
 (gr_line (start 88 109) (end 88.5 110) (stroke (width 0.05) (type default)) (layer "Edge.Cuts"))
 (gr_line (start 88 121) (end 88 125) (stroke (width 0.05) (type default)) (layer "Edge.Cuts"))
 (gr_line (start 88 125) (end 87 125) (stroke (width 0.05) (type default)) (layer "Edge.Cuts"))
 (gr_line (start 88.5 108) (end 89 107) (stroke (width 0.05) (type default)) (layer "Edge.Cuts"))
 (gr_line (start 88.5 110) (end 89 110) (stroke (width 0.05) (type default)) (layer "Edge.Cuts"))
 (gr_line (start 89 107) (end 89.5 107) (stroke (width 0.05) (type default)) (layer "Edge.Cuts"))
 (gr_line (start 89 110) (end 89.5 109) (stroke (width 0.05) (type default)) (layer "Edge.Cuts"))
 (gr_line (start 89.5 107) (end 90 108) (stroke (width 0.05) (type default)) (layer "Edge.Cuts"))
 (gr_line (start 89.5 109) (end 90 110) (stroke (width 0.05) (type default)) (layer "Edge.Cuts"))
 (gr_line (start 90 108) (end 90.5 107) (stroke (width 0.05) (type default)) (layer "Edge.Cuts"))
 (gr_line (start 90 110) (end 90.5 110) (stroke (width 0.05) (type default)) (layer "Edge.Cuts"))
 (gr_line (start 90.5 107) (end 91 107) (stroke (width 0.05) (type default)) (layer "Edge.Cuts"))
 (gr_line (start 90.5 110) (end 91 109) (stroke (width 0.05) (type default)) (layer "Edge.Cuts"))
 (gr_line (start 91 107) (end 91.5 108) (stroke (width 0.05) (type default)) (layer "Edge.Cuts"))
 (gr_line (start 91 109) (end 91.5 110) (stroke (width 0.05) (type default)) (layer "Edge.Cuts"))
 (gr_line (start 91.5 70) (end 76.5 70) (stroke (width 0.05) (type default)) (layer "Edge.Cuts"))
 (gr_line (start 91.5 74.5) (end 91.5 70) (stroke (width 0.05) (type default)) (layer "Edge.Cuts"))
 (gr_line (start 91.5 108) (end 92 107) (stroke (width 0.05) (type default)) (layer "Edge.Cuts"))
 (gr_line (start 91.5 110) (end 92 110) (stroke (width 0.05) (type default)) (layer "Edge.Cuts"))
 (gr_line (start 92 107) (end 92.5 107) (stroke (width 0.05) (type default)) (layer "Edge.Cuts"))
 (gr_line (start 92 110) (end 92.5 109) (stroke (width 0.05) (type default)) (layer "Edge.Cuts"))
 (gr_line (start 92.5 107) (end 93 108) (stroke (width 0.05) (type default)) (layer "Edge.Cuts"))
 (gr_line (start 92.5 109) (end 93 110) (stroke (width 0.05) (type default)) (layer "Edge.Cuts"))
 (gr_line (start 93 108) (end 93.5 107) (stroke (width 0.05) (type default)) (layer "Edge.Cuts"))
 (gr_line (start 93 110) (end 93.5 110) (stroke (width 0.05) (type default)) (layer "Edge.Cuts"))
 (gr_line (start 93.5 107) (end 94 107) (stroke (width 0.05) (type default)) (layer "Edge.Cuts"))
 (gr_line (start 93.5 110) (end 94 109) (stroke (width 0.05) (type default)) (layer "Edge.Cuts"))
 (gr_line (start 94 107) (end 94.5 108) (stroke (width 0.05) (type default)) (layer "Edge.Cuts"))
 (gr_line (start 94 109) (end 94.5 110) (stroke (width 0.05) (type default)) (layer "Edge.Cuts"))
 (gr_line (start 94.5 108) (end 95 107) (stroke (width 0.05) (type default)) (layer "Edge.Cuts"))
 (gr_line (start 94.5 110) (end 95 110) (stroke (width 0.05) (type default)) (layer "Edge.Cuts"))
 (gr_line (start 95 107) (end 95.5 107) (stroke (width 0.05) (type default)) (layer "Edge.Cuts"))
 (gr_line (start 95 110) (end 95.5 109) (stroke (width 0.05) (type default)) (layer "Edge.Cuts"))
 (gr_line (start 95 112) (end 95 113.5) (stroke (width 0.05) (type default)) (layer "Edge.Cuts"))
 (gr_line (start 95 113.5) (end 79.5 113.5) (stroke (width 0.05) (type default)) (layer "Edge.Cuts"))
 (gr_line (start 95.5 107) (end 96 108) (stroke (width 0.05) (type default)) (layer "Edge.Cuts"))
 (gr_line (start 95.5 109) (end 96 110) (stroke (width 0.05) (type default)) (layer "Edge.Cuts"))
 (gr_line (start 96 108) (end 96.5 107) (stroke (width 0.05) (type default)) (layer "Edge.Cuts"))
 (gr_line (start 96 110) (end 96.5 110) (stroke (width 0.05) (type default)) (layer "Edge.Cuts"))
 (gr_line (start 96.5 110) (end 97 109) (stroke (width 0.05) (type default)) (layer "Edge.Cuts"))
 (gr_line (start 97 107) (end 96.5 107) (stroke (width 0.05) (type default)) (layer "Edge.Cuts"))
 (gr_line (start 97 107) (end 97.5 108) (stroke (width 0.05) (type default)) (layer "Edge.Cuts"))
 (gr_line (start 97 109) (end 97.5 110) (stroke (width 0.05) (type default)) (layer "Edge.Cuts"))
 (gr_line (start 97.5 108) (end 98 107) (stroke (width 0.05) (type default)) (layer "Edge.Cuts"))
 (gr_line (start 97.5 110) (end 98 110) (stroke (width 0.05) (type default)) (layer "Edge.Cuts"))
 (gr_line (start 98 107) (end 98.5 107) (stroke (width 0.05) (type default)) (layer "Edge.Cuts"))
 (gr_line (start 98 110) (end 98.5 109) (stroke (width 0.05) (type default)) (layer "Edge.Cuts"))
 (gr_line (start 98.5 107) (end 99 108) (stroke (width 0.05) (type default)) (layer "Edge.Cuts"))
 (gr_line (start 98.5 109) (end 99 110) (stroke (width 0.05) (type default)) (layer "Edge.Cuts"))
 (gr_line (start 99 108) (end 99.5 107) (stroke (width 0.05) (type default)) (layer "Edge.Cuts"))
 (gr_line (start 99 110) (end 99.5 110) (stroke (width 0.05) (type default)) (layer "Edge.Cuts"))
 (gr_line (start 99.5 107) (end 100 107) (stroke (width 0.05) (type default)) (layer "Edge.Cuts"))
 (gr_line (start 99.5 110) (end 100 109) (stroke (width 0.05) (type default)) (layer "Edge.Cuts"))
 (gr_line (start 100 107) (end 100.5 108) (stroke (width 0.05) (type default)) (layer "Edge.Cuts"))
 (gr_line (start 100 109) (end 100.5 110) (stroke (width 0.05) (type default)) (layer "Edge.Cuts"))
 (gr_line (start 100.5 108) (end 101 107) (stroke (width 0.05) (type default)) (layer "Edge.Cuts"))
 (gr_line (start 100.5 110) (end 101 110) (stroke (width 0.05) (type default)) (layer "Edge.Cuts"))
 (gr_line (start 101 107) (end 101.5 107) (stroke (width 0.05) (type default)) (layer "Edge.Cuts"))
 (gr_line (start 101 110) (end 101.5 109) (stroke (width 0.05) (type default)) (layer "Edge.Cuts"))
 (gr_line (start 101.5 107) (end 102 108) (stroke (width 0.05) (type default)) (layer "Edge.Cuts"))
 (gr_line (start 101.5 109) (end 102 110) (stroke (width 0.05) (type default)) (layer "Edge.Cuts"))
 (gr_line (start 102 108) (end 102.5 107) (stroke (width 0.05) (type default)) (layer "Edge.Cuts"))
 (gr_line (start 102 110) (end 102.5 110) (stroke (width 0.05) (type default)) (layer "Edge.Cuts"))
 (gr_line (start 102.5 107) (end 103 107) (stroke (width 0.05) (type default)) (layer "Edge.Cuts"))
 (gr_line (start 102.5 110) (end 103 109) (stroke (width 0.05) (type default)) (layer "Edge.Cuts"))
 (gr_line (start 102.5 111) (end 102.5 112) (stroke (width 0.05) (type default)) (layer "Edge.Cuts"))
 (gr_line (start 102.5 112) (end 95 112) (stroke (width 0.05) (type default)) (layer "Edge.Cuts"))
 (gr_line (start 103 107) (end 103.5 108) (stroke (width 0.05) (type default)) (layer "Edge.Cuts"))
 (gr_line (start 103 109) (end 103.5 110) (stroke (width 0.05) (type default)) (layer "Edge.Cuts"))
 (gr_line (start 103.5 108) (end 104 107) (stroke (width 0.05) (type default)) (layer "Edge.Cuts"))
 (gr_line (start 103.5 110) (end 104 110) (stroke (width 0.05) (type default)) (layer "Edge.Cuts"))
 (gr_line (start 104 107) (end 104 104.5) (stroke (width 0.05) (type default)) (layer "Edge.Cuts"))
 (gr_line (start 104 110) (end 104 111) (stroke (width 0.05) (type default)) (layer "Edge.Cuts"))
 (gr_line (start 104 111) (end 102.5 111) (stroke (width 0.05) (type default)) (layer "Edge.Cuts"))
 (gr_line (start 106.5 104.5) (end 104 104.5) (stroke (width 0.05) (type default)) (layer "Edge.Cuts"))
 (gr_line (start 106.5 104.5) (end 106.5 98.5) (stroke (width 0.05) (type default)) (layer "Edge.Cuts"))
 (gr_line (start 110 74.5) (end 91.5 74.5) (stroke (width 0.05) (type default)) (layer "Edge.Cuts"))
 (gr_line (start 110 98.5) (end 106.5 98.5) (stroke (width 0.05) (type default)) (layer "Edge.Cuts"))
 (gr_line (start 110 98.5) (end 110 74.5) (stroke (width 0.05) (type default)) (layer "Edge.Cuts"))
 (segment (start 69.739 103.064) (end 67.054 105.749) (width 0.2) (layer "F.Cu") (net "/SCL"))
 (segment (start 85.524642 103.064) (end 69.739 103.064) (width 0.2) (layer "F.Cu") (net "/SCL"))
 (segment (start 84.335 96.66) (end 86.01 98.335) (width 0.2) (layer "F.Cu") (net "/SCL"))
 (segment (start 86.01 102.578642) (end 85.524642 103.064) (width 0.2) (layer "F.Cu") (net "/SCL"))
 (segment (start 86.01 98.335) (end 86.01 102.578642) (width 0.2) (layer "F.Cu") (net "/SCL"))
 (segment (start 71.063 99.2) (end 64.514 105.749) (width 0.2) (layer "F.Cu") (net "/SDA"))
 (segment (start 84.335 99.2) (end 71.063 99.2) (width 0.2) (layer "F.Cu") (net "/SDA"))
 (segment (start 68.5 74.5) (end 68.5 70.5) (width 0.2) (layer "F.Cu") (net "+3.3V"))
 (segment (start 68.5 70.5) (end 67.5 69.5) (width 0.2) (layer "F.Cu") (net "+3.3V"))
 (segment (start 60.96 69.5) (end 65.96 74.5) (width 0.2) (layer "F.Cu") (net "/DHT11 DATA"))
 (segment (start 80.5 89.04) (end 84.335 89.04) (width 0.2) (layer "F.Cu") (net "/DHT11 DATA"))
 (segment (start 59.88 69.5) (end 60.96 69.5) (width 0.2) (layer "F.Cu") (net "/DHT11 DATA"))
 (segment (start 65.96 74.5) (end 80.5 89.04) (width 0.2) (layer "F.Cu") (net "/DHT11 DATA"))
 (segment (start 42.46 89.92) (end 44.66 92.12) (width 0.2) (layer "F.Cu") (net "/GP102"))
 (segment (start 43 90) (end 43 89.5) (width 0.2) (layer "F.Cu") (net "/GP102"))
 (segment (start 83.795 92.12) (end 84.335 91.58) (width 0.2) (layer "F.Cu") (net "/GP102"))
 (segment (start 44.66 92.12) (end 83.795 92.12) (width 0.2) (layer "F.Cu") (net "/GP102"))
 (segment (start 48 112.5) (end 48 110.912862) (width 0.2) (layer "F.Cu") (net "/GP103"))
 (segment (start 64.792862 94.12) (end 84.335 94.12) (width 0.2) (layer "F.Cu") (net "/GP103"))
 (segment (start 48 110.912862) (end 64.792862 94.12) (width 0.2) (layer "F.Cu") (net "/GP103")))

